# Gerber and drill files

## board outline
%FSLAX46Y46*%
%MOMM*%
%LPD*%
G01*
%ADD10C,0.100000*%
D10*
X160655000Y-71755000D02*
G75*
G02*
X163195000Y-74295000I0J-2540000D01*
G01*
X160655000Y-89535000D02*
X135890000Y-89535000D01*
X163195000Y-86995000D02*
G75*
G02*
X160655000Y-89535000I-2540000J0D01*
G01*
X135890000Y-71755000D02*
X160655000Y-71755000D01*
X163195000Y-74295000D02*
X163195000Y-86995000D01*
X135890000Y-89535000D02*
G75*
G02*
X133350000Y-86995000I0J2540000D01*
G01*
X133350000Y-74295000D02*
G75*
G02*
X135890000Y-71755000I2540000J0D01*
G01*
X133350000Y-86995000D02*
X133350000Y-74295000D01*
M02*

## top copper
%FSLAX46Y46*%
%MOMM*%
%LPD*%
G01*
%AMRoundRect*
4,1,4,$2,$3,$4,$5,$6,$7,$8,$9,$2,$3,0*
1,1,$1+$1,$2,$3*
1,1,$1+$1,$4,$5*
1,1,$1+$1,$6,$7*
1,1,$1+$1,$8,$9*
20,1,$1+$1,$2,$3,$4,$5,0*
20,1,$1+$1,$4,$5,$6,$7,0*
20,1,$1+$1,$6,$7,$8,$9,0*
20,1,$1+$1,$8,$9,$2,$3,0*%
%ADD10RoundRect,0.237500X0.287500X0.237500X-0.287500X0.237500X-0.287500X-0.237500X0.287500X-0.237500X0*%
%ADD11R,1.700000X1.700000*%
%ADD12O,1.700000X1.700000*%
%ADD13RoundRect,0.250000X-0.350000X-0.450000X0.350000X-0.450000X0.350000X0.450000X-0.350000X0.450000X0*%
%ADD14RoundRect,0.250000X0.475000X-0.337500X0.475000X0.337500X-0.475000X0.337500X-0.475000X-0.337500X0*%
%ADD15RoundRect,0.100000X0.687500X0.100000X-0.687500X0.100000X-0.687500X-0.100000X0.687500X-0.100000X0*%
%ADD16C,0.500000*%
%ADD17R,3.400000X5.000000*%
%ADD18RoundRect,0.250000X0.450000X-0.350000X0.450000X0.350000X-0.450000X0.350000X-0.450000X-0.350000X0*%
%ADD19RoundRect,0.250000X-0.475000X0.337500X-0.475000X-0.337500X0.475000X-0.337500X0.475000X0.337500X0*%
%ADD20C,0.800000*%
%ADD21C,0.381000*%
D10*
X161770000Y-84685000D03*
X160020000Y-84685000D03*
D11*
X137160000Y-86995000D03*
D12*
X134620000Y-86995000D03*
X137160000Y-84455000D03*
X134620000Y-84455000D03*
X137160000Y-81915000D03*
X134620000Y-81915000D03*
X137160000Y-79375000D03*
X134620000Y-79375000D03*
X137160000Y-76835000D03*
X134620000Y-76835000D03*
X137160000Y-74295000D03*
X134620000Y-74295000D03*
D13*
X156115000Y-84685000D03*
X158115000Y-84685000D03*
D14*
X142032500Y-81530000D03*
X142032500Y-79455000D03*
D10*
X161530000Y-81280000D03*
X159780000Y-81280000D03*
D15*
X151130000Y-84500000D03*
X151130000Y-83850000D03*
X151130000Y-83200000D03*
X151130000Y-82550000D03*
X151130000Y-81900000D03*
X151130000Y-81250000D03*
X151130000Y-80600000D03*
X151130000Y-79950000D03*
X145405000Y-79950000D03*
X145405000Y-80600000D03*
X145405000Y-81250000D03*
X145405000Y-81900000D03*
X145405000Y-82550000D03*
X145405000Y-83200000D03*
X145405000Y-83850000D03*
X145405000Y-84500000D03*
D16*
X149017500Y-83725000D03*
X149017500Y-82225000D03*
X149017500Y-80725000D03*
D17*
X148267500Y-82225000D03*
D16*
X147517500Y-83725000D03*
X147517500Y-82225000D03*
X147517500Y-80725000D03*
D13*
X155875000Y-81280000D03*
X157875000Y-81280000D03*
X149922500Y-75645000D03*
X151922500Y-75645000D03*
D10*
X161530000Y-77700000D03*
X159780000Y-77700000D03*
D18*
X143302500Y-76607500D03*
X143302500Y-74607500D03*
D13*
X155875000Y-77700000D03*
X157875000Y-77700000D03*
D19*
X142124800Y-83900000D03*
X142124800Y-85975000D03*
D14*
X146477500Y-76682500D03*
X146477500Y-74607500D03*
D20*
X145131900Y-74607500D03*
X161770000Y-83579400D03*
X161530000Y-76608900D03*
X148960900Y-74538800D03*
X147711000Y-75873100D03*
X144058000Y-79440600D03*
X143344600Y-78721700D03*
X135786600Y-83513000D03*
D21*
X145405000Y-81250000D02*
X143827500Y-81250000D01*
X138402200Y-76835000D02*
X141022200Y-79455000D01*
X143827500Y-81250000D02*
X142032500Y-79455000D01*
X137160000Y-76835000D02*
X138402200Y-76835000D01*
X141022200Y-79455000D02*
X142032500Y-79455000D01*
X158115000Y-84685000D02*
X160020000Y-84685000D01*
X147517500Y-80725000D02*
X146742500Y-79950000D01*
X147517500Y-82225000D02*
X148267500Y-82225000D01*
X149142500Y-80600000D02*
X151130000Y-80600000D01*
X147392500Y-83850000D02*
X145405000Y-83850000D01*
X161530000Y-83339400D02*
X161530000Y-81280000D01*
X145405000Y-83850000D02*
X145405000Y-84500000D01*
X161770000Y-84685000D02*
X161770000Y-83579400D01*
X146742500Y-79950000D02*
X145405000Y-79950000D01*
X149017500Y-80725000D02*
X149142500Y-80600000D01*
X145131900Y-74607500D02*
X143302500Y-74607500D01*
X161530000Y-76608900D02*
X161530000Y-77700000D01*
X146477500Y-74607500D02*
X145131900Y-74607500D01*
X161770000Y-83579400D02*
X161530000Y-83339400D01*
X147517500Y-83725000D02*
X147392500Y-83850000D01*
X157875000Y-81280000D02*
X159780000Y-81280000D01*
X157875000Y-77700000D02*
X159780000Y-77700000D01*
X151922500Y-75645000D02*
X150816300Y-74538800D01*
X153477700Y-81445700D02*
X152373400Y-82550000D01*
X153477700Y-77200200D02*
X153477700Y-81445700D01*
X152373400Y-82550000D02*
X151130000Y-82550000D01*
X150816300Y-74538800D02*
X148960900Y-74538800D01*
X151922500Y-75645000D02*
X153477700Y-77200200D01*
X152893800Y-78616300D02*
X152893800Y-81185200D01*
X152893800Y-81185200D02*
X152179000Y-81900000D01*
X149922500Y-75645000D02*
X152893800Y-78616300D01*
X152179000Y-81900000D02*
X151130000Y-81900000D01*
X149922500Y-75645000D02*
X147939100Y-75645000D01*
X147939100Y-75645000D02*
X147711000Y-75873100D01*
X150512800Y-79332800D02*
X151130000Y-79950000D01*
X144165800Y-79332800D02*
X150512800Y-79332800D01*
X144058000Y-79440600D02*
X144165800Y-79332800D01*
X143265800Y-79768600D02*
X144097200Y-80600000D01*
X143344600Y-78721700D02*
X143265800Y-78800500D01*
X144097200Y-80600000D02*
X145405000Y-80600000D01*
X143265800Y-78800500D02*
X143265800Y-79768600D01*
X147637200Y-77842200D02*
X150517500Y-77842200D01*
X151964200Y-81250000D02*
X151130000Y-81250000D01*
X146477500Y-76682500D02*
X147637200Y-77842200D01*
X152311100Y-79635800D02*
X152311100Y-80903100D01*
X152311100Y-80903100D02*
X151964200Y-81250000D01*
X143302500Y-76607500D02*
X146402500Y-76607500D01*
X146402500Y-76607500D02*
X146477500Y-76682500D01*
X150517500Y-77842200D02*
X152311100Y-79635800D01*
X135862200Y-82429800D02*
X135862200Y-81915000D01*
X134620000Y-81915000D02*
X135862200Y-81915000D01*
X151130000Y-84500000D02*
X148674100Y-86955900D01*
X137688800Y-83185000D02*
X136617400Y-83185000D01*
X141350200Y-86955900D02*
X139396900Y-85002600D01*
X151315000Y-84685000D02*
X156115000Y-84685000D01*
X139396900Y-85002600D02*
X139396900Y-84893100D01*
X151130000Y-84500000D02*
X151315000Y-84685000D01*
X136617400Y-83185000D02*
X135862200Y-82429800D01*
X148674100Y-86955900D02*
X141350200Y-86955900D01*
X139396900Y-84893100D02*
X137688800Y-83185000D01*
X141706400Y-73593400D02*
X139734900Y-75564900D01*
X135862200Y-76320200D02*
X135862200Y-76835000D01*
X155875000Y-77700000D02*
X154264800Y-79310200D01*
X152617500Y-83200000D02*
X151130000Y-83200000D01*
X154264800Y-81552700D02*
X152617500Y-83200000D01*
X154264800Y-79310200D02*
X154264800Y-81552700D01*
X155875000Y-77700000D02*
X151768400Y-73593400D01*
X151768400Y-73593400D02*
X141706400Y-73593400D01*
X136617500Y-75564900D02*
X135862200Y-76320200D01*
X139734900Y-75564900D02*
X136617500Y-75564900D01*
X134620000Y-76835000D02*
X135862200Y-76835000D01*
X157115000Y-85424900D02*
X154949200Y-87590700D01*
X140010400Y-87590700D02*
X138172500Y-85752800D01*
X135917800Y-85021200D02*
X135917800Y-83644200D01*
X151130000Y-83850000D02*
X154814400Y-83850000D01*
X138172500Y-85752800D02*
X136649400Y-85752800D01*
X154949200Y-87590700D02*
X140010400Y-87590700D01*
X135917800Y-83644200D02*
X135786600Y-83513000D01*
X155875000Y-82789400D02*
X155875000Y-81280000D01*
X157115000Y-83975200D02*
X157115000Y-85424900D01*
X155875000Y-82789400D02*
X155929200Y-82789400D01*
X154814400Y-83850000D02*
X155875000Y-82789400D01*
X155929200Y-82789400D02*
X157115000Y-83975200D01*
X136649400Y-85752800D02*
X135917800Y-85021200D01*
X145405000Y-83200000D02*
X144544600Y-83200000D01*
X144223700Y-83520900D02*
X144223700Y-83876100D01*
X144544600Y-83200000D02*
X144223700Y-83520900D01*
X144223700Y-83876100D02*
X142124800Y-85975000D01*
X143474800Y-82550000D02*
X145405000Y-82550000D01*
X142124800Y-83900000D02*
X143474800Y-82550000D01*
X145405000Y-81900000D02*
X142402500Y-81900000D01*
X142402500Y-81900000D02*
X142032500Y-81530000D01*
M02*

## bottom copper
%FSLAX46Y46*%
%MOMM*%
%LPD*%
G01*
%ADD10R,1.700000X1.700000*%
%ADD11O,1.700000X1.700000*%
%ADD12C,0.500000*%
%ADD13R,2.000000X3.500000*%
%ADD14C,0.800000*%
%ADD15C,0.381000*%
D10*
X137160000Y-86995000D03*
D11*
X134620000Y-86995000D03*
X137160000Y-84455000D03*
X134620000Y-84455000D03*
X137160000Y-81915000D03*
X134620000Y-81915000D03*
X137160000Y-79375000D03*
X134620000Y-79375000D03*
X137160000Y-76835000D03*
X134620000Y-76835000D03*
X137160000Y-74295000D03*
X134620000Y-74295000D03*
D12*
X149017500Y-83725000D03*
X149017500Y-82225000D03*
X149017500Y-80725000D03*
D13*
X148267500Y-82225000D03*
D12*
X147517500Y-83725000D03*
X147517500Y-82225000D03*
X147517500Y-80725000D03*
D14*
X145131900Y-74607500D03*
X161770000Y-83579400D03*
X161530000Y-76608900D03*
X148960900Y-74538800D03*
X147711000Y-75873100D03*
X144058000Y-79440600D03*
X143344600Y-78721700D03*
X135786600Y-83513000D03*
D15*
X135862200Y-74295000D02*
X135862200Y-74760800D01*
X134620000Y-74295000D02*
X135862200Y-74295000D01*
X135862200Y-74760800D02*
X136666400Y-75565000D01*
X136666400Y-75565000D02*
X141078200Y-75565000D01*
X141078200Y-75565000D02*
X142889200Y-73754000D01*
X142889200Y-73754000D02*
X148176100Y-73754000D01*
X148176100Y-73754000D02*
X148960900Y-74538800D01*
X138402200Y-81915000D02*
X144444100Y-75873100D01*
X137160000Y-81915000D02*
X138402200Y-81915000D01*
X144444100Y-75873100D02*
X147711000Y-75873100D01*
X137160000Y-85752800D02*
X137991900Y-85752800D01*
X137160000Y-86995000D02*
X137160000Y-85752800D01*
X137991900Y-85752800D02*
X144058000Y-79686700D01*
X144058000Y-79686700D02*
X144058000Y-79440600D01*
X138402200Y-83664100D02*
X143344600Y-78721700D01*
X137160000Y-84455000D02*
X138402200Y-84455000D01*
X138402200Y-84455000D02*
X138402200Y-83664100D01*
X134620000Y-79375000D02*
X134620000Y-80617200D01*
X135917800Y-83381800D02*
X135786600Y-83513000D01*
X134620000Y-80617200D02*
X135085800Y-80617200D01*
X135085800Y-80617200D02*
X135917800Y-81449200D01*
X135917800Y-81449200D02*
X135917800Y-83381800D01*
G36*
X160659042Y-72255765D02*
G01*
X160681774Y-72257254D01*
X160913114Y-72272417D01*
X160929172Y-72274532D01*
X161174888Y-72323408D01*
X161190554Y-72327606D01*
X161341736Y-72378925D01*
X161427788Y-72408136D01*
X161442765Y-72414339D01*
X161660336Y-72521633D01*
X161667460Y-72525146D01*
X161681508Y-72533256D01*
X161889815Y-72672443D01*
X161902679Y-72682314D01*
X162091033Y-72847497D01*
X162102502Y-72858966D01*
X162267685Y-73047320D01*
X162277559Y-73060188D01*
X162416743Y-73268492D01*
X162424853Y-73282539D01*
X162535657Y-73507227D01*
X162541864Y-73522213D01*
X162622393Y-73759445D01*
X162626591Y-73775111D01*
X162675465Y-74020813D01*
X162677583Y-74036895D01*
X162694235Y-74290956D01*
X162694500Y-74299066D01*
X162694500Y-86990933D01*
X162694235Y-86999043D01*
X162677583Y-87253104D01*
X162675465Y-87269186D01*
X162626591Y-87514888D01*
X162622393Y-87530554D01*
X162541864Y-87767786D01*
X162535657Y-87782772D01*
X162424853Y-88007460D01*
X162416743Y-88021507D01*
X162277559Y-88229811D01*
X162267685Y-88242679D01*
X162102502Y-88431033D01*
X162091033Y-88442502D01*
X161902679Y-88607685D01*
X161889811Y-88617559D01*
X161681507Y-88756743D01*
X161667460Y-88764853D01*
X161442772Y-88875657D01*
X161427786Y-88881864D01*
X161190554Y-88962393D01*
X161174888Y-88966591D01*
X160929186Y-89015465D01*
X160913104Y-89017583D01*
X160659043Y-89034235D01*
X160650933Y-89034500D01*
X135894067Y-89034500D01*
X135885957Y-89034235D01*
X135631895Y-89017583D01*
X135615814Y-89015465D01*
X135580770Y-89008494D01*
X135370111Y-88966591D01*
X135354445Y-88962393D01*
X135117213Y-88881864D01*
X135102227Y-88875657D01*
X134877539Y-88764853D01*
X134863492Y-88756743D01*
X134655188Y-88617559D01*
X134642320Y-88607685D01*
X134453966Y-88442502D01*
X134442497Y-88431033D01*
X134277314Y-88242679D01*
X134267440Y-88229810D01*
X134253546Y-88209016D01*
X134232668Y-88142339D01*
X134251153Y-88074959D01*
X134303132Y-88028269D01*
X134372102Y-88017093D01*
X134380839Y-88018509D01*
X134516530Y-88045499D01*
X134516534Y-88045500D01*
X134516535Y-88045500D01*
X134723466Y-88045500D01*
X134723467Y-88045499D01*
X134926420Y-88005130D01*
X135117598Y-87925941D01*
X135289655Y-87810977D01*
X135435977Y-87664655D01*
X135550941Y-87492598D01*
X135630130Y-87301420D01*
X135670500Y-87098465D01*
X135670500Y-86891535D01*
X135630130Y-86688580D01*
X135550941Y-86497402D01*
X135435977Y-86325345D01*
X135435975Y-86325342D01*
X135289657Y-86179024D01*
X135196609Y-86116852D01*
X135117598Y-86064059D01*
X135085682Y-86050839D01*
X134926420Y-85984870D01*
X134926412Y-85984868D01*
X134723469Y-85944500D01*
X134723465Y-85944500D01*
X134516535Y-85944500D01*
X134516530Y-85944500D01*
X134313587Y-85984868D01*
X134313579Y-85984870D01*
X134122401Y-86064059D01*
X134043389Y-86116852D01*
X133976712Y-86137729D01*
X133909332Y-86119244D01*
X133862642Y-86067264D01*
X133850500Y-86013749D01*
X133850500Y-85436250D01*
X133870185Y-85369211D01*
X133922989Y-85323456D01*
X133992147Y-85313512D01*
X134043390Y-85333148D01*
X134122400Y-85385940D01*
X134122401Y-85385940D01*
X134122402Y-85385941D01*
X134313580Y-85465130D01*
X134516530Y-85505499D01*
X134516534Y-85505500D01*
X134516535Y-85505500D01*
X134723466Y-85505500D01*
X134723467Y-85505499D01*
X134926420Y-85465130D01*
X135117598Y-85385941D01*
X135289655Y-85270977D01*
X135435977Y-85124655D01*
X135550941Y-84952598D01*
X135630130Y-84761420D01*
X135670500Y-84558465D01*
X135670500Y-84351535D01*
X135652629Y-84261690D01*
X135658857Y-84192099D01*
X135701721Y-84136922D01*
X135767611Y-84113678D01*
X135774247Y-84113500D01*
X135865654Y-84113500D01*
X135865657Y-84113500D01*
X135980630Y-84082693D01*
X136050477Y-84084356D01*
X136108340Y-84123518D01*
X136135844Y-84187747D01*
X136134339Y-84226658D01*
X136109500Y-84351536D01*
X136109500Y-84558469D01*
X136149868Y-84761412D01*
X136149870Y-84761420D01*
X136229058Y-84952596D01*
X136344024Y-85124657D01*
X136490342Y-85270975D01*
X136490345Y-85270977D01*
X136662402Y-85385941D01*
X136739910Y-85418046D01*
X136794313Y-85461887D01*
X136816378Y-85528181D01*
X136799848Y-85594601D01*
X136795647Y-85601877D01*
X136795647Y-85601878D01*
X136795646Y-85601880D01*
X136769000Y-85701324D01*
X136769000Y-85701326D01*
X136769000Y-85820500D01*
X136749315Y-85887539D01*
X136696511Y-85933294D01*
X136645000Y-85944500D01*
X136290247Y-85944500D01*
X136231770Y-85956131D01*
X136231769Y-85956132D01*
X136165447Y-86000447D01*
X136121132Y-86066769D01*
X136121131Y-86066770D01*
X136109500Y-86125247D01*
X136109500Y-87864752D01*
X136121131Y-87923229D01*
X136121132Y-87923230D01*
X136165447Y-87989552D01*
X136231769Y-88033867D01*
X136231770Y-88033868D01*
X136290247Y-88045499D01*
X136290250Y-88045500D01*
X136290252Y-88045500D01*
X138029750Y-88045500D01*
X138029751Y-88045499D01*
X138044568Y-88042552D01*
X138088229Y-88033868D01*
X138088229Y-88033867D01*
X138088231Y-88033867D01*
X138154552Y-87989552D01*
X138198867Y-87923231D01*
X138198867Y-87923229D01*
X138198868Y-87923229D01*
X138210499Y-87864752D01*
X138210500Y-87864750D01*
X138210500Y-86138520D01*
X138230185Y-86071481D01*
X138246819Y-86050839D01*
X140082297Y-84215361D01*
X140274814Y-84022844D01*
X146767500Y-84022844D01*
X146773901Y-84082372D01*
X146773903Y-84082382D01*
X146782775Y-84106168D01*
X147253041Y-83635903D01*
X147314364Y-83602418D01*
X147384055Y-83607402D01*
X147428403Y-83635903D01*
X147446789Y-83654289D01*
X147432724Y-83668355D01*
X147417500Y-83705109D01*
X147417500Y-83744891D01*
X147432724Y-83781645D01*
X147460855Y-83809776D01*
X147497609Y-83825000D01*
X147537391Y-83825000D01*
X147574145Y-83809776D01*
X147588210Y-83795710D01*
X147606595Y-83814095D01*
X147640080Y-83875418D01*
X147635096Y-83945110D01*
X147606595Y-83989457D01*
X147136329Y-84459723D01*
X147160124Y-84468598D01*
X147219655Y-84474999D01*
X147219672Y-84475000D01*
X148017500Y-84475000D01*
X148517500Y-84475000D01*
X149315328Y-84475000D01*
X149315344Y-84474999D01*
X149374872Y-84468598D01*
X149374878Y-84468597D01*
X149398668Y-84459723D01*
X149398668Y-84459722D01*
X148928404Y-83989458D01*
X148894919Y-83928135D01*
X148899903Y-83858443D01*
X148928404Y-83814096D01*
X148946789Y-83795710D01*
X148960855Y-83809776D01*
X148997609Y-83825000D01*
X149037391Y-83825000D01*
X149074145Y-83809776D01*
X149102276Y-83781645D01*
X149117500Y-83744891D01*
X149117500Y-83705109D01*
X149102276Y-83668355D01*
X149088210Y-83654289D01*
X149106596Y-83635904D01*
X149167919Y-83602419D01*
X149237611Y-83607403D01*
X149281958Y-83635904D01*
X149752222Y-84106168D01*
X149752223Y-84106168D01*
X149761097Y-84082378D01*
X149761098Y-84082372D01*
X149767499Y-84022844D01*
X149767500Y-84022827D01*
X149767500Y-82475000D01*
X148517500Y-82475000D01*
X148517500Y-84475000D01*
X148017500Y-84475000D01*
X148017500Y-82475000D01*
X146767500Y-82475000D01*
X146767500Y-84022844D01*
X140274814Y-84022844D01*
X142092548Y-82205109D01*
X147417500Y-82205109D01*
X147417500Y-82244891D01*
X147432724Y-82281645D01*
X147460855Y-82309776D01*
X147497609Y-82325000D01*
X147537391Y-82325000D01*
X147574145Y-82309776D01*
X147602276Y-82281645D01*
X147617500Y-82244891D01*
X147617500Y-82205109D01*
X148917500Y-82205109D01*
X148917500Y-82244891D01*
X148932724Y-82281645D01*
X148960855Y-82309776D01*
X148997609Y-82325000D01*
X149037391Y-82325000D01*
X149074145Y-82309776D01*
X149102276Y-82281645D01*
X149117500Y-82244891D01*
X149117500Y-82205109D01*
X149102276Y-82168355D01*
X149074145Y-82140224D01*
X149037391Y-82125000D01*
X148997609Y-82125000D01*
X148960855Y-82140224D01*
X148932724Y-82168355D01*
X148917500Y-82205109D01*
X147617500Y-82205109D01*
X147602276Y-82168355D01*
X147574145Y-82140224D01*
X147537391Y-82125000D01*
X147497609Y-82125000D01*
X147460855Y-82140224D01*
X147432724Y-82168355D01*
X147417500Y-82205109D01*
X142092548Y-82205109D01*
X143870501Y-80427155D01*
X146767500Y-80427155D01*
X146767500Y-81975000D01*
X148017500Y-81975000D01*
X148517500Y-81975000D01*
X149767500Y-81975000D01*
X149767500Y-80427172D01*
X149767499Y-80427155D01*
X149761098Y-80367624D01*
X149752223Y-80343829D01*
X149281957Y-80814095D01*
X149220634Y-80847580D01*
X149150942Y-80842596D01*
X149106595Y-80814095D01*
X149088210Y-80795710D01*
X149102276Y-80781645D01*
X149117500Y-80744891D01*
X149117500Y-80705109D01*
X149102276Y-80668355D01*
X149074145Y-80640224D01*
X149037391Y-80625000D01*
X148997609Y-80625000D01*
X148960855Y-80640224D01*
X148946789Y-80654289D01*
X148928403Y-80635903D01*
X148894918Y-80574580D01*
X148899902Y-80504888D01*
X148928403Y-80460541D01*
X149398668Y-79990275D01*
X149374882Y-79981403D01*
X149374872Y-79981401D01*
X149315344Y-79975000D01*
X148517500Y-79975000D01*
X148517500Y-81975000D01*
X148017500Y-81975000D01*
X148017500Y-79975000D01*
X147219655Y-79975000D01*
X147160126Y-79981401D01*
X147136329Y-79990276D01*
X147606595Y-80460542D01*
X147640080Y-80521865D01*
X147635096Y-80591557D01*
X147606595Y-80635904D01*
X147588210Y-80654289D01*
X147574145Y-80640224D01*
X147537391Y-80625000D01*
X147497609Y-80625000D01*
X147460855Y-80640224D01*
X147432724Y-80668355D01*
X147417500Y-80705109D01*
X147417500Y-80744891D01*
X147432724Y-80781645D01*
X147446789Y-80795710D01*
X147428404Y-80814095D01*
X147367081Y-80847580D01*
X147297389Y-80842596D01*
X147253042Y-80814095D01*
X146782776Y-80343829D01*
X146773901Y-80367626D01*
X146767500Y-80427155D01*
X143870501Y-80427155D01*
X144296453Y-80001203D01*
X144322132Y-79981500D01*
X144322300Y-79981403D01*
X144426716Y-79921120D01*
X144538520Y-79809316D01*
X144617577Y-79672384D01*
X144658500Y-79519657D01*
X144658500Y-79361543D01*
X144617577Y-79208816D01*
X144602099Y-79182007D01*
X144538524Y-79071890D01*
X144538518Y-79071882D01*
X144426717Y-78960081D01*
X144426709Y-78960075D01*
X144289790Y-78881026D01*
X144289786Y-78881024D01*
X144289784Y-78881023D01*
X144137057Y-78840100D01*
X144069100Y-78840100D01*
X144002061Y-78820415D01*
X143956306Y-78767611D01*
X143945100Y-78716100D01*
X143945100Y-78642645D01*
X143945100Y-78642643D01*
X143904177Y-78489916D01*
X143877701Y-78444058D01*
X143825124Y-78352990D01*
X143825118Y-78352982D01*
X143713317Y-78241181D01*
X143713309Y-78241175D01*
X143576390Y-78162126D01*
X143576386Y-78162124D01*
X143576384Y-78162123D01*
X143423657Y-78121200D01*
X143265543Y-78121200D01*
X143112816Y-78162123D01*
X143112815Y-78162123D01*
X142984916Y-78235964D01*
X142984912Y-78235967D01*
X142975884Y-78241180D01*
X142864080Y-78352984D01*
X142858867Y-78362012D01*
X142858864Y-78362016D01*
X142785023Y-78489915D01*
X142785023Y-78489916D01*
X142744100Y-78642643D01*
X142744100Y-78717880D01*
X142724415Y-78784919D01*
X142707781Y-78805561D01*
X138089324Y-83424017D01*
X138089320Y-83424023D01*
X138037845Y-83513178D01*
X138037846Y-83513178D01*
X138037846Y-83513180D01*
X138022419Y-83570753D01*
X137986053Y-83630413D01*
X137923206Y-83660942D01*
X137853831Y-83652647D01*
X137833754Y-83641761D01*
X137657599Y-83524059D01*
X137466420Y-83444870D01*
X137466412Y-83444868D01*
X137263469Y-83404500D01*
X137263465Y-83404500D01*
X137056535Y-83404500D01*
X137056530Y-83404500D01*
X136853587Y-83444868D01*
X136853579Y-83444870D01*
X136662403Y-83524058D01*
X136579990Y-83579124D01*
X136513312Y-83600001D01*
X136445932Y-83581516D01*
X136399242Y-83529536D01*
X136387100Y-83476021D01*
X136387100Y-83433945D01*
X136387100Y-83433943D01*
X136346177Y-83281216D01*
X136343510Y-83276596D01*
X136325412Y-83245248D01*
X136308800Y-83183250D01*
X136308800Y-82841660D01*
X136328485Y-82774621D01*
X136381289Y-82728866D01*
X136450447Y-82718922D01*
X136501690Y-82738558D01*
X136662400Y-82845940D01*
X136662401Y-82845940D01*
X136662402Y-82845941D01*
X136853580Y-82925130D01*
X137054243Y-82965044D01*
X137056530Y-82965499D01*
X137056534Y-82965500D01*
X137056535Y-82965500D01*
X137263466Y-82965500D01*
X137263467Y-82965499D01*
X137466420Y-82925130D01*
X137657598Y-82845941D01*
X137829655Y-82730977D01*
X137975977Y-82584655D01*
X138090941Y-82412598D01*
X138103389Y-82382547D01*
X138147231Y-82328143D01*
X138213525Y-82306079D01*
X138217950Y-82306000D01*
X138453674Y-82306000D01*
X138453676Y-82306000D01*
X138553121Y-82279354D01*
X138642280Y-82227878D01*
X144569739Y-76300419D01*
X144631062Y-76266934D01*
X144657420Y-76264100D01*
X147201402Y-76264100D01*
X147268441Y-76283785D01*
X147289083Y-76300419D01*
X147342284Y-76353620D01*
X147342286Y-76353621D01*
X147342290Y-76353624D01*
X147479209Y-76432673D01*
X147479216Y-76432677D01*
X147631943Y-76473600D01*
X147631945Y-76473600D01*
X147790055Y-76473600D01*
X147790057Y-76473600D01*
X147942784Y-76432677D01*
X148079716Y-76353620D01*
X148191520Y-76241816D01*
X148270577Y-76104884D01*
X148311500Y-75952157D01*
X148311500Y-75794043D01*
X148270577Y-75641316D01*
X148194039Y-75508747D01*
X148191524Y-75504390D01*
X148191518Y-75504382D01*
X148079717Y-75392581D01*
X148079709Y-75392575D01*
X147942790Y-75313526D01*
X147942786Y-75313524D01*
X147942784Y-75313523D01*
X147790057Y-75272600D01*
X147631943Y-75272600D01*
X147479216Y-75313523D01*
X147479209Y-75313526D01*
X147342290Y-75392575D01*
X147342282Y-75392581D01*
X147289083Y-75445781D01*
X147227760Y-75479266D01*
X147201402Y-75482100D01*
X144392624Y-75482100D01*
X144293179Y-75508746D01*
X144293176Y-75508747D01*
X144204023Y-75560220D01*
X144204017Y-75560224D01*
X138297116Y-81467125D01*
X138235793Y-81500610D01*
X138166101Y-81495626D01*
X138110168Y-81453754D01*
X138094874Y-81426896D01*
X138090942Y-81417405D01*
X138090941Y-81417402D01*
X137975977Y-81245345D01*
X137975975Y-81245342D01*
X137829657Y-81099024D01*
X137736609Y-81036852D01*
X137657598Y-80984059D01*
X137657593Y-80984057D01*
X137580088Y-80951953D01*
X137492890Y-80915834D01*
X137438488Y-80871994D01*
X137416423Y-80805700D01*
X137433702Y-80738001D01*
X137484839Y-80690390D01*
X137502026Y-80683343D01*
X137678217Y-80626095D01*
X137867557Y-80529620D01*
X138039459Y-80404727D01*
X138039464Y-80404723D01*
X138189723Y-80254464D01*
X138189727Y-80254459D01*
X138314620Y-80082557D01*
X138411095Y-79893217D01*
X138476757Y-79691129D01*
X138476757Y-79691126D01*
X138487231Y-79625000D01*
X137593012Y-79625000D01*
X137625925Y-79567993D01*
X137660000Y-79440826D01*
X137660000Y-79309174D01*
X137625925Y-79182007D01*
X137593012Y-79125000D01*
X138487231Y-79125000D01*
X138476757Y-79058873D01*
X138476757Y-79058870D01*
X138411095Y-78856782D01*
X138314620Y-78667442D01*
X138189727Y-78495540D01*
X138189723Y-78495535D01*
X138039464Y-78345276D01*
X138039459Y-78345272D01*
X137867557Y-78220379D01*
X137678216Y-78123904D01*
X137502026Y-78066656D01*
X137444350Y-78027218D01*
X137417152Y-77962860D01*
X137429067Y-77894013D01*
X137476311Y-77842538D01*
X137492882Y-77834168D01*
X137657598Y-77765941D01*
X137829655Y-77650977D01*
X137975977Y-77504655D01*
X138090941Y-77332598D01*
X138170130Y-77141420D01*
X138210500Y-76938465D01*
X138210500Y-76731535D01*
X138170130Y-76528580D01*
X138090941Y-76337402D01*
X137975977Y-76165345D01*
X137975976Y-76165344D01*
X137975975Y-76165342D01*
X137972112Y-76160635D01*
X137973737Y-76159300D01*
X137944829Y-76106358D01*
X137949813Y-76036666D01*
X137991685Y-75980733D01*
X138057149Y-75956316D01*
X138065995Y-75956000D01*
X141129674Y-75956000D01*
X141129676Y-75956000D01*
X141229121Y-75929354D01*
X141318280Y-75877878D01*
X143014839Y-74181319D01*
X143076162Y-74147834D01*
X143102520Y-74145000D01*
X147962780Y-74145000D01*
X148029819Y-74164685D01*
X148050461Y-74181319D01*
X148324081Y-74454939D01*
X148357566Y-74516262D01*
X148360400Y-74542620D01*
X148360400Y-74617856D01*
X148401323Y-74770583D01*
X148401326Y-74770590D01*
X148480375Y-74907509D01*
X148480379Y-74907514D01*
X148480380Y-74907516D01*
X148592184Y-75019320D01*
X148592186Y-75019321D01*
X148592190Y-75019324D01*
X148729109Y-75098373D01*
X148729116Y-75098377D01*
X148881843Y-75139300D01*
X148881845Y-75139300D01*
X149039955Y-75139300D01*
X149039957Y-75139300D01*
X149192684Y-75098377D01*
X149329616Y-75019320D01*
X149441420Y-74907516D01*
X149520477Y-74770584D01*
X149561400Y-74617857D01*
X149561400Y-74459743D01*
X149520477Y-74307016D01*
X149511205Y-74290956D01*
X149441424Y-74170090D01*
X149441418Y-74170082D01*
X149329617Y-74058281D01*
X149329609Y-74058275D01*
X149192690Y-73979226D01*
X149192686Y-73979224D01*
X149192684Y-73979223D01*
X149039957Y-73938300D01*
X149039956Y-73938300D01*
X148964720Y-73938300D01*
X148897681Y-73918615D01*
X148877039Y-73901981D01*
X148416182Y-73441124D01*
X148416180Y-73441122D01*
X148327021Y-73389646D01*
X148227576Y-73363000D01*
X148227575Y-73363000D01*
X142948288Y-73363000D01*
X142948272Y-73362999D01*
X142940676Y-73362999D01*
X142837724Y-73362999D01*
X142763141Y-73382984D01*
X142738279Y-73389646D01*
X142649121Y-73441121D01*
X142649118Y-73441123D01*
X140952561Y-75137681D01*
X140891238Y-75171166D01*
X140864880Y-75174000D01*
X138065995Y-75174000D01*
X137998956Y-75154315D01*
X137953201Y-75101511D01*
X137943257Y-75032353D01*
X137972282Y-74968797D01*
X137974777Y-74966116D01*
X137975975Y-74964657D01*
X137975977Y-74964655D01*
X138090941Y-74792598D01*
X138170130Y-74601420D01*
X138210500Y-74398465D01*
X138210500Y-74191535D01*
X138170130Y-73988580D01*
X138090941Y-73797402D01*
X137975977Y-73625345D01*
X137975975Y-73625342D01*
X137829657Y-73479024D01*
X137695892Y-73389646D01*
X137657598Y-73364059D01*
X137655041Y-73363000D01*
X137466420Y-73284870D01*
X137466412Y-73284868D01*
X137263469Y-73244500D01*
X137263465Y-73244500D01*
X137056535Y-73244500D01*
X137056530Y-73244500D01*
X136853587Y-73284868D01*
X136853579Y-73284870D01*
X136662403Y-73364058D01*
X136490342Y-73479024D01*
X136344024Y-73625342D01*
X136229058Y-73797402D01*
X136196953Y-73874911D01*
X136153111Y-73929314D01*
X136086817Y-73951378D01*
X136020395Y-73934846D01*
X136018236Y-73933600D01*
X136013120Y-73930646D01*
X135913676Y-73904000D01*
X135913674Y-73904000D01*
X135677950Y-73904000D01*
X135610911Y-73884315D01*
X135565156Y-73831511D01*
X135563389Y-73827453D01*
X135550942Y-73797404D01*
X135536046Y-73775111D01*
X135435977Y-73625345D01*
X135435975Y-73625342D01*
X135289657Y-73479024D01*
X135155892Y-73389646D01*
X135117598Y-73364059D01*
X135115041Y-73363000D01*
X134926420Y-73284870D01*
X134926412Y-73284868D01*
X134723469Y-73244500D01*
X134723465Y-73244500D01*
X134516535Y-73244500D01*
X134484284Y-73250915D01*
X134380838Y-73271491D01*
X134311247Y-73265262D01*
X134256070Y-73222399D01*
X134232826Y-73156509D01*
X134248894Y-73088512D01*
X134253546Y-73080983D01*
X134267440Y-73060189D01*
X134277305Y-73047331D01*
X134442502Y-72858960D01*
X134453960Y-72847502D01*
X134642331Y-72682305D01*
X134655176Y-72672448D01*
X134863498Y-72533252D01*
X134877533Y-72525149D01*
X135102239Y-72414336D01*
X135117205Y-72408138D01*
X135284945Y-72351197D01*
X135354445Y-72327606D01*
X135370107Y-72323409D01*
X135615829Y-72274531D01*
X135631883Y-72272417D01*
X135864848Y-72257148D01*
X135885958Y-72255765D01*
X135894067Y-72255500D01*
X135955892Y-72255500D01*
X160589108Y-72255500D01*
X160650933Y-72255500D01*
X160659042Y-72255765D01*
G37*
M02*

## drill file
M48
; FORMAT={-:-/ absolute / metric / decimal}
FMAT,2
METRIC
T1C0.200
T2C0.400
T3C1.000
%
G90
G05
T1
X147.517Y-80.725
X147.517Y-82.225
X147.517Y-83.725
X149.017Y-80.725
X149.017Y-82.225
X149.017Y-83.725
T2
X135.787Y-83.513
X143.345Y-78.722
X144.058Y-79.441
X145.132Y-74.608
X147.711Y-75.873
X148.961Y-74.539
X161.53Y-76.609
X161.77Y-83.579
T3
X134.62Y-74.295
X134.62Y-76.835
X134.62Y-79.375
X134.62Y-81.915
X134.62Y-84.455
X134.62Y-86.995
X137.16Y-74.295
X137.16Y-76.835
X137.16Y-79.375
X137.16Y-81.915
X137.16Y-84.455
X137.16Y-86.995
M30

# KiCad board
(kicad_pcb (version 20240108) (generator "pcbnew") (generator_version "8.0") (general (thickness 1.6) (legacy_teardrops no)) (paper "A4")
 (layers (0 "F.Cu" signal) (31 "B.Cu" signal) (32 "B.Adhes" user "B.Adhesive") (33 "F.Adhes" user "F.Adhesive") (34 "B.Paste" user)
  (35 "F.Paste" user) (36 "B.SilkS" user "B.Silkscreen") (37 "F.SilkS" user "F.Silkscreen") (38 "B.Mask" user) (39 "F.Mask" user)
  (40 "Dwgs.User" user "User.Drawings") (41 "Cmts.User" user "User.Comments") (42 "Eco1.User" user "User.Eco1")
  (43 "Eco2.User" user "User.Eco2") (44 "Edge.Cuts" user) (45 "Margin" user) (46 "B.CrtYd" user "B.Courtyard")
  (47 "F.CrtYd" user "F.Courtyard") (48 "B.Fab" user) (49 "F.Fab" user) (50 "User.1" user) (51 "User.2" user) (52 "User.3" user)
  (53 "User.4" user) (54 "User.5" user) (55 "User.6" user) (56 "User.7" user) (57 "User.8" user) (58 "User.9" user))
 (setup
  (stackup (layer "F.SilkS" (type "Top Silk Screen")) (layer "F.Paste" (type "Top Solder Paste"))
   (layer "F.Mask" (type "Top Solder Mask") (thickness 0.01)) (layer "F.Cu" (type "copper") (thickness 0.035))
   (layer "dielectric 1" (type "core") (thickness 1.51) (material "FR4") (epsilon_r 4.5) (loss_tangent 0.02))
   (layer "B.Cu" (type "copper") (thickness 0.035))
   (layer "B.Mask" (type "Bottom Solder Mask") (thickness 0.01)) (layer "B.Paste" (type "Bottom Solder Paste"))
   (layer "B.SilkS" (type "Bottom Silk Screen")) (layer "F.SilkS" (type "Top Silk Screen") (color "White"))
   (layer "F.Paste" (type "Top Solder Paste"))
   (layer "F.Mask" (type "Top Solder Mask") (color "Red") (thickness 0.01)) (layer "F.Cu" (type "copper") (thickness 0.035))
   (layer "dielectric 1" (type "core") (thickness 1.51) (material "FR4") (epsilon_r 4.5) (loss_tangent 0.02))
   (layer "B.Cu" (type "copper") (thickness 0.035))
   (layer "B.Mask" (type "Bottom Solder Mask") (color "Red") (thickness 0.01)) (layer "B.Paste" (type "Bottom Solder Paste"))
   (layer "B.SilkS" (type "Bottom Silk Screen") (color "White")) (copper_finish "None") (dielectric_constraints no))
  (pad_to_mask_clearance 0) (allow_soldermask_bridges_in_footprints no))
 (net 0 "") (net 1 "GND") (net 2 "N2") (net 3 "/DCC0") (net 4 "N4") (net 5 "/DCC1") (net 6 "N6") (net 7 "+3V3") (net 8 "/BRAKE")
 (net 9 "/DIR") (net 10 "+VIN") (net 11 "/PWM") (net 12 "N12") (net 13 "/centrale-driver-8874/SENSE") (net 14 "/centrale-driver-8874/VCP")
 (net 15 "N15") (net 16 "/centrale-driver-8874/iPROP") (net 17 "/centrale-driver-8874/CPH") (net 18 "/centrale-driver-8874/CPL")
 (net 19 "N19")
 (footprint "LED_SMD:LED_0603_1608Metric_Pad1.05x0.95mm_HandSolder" (layer "F.Cu") (at 160.895 84.685 180)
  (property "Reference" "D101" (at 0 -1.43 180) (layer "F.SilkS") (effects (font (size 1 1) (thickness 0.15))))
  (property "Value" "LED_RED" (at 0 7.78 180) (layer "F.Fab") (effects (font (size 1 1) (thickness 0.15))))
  (pad "1" smd roundrect (at -0.875 0 180) (size 1.05 0.95) (layers "F.Cu" "F.Paste" "F.Mask") (roundrect_rratio 0.25) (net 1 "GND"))
  (pad "2" smd roundrect (at 0.875 0 180) (size 1.05 0.95) (layers "F.Cu" "F.Paste" "F.Mask") (roundrect_rratio 0.25) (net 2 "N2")))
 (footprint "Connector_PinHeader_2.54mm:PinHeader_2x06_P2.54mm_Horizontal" (layer "F.Cu") (at 137.16 86.995 180)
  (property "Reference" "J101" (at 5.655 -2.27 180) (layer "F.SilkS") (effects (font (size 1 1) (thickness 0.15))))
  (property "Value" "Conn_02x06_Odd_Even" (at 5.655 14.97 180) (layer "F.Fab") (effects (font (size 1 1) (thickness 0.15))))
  (pad "1" thru_hole rect (at 0 0 180) (size 1.7 1.7) (drill 1) (layers "*.Cu" "*.Mask") (remove_unused_layers no) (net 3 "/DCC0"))
  (pad "2" thru_hole oval (at 2.54 0 180) (size 1.7 1.7) (drill 1) (layers "*.Cu" "*.Mask") (remove_unused_layers no) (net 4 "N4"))
  (pad "3" thru_hole oval (at 0 2.54 180) (size 1.7 1.7) (drill 1) (layers "*.Cu" "*.Mask") (remove_unused_layers no) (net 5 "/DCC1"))
  (pad "4" thru_hole oval (at 2.54 2.54 180) (size 1.7 1.7) (drill 1) (layers "*.Cu" "*.Mask") (remove_unused_layers no) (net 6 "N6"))
  (pad "5" thru_hole oval (at 0 5.08 180) (size 1.7 1.7) (drill 1) (layers "*.Cu" "*.Mask") (remove_unused_layers no) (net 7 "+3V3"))
  (pad "6" thru_hole oval (at 2.54 5.08 180) (size 1.7 1.7) (drill 1) (layers "*.Cu" "*.Mask") (remove_unused_layers no) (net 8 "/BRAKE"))
  (pad "7" thru_hole oval (at 0 7.62 180) (size 1.7 1.7) (drill 1) (layers "*.Cu" "*.Mask") (remove_unused_layers no) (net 1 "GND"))
  (pad "8" thru_hole oval (at 2.54 7.62 180) (size 1.7 1.7) (drill 1) (layers "*.Cu" "*.Mask") (remove_unused_layers no) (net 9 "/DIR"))
  (pad "9" thru_hole oval (at 0 10.16 180) (size 1.7 1.7) (drill 1) (layers "*.Cu" "*.Mask") (remove_unused_layers no) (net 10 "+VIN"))
  (pad "10" thru_hole oval (at 2.54 10.16 180) (size 1.7 1.7) (drill 1) (layers "*.Cu" "*.Mask") (remove_unused_layers no) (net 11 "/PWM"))
  (pad "11" thru_hole oval (at 0 12.7 180) (size 1.7 1.7) (drill 1) (layers "*.Cu" "*.Mask") (remove_unused_layers no) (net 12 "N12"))
  (pad "12" thru_hole oval (at 2.54 12.7 180) (size 1.7 1.7) (drill 1) (layers "*.Cu" "*.Mask") (remove_unused_layers no)
   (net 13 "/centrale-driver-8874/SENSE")))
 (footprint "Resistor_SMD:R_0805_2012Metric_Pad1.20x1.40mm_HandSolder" (layer "F.Cu") (at 157.115 84.685)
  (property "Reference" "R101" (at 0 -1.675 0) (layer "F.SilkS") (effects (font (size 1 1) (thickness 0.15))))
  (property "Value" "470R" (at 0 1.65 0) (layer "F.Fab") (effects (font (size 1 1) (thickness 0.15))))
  (pad "1" smd roundrect (at -1 0) (size 1.2 1.4) (layers "F.Cu" "F.Paste" "F.Mask") (roundrect_rratio 0.208333) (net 8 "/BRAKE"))
  (pad "2" smd roundrect (at 1 0) (size 1.2 1.4) (layers "F.Cu" "F.Paste" "F.Mask") (roundrect_rratio 0.208333) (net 2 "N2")))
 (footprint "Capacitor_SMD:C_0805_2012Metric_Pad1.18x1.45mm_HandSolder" (layer "F.Cu") (at 142.0325 80.4925 90)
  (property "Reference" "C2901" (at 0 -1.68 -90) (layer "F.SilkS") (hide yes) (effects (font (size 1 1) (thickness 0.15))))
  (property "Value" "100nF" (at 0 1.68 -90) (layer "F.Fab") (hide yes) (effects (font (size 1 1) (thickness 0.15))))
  (pad "1" smd roundrect (at -1.0375 0 90) (size 1.175 1.45) (layers "F.Cu" "F.Paste" "F.Mask") (roundrect_rratio 0.212766)
   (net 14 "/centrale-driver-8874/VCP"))
  (pad "2" smd roundrect (at 1.0375 0 90) (size 1.175 1.45) (layers "F.Cu" "F.Paste" "F.Mask") (roundrect_rratio 0.212766) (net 10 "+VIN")))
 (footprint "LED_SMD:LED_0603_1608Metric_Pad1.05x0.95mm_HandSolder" (layer "F.Cu") (at 160.655 81.28 180)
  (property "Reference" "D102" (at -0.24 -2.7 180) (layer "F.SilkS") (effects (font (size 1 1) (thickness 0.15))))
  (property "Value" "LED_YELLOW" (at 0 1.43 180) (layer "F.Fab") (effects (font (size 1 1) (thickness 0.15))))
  (pad "1" smd roundrect (at -0.875 0 180) (size 1.05 0.95) (layers "F.Cu" "F.Paste" "F.Mask") (roundrect_rratio 0.25) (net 1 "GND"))
  (pad "2" smd roundrect (at 0.875 0 180) (size 1.05 0.95) (layers "F.Cu" "F.Paste" "F.Mask") (roundrect_rratio 0.25) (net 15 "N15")))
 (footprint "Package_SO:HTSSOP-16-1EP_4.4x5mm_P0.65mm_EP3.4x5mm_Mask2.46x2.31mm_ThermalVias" (layer "F.Cu") (at 148.2675 82.225 180)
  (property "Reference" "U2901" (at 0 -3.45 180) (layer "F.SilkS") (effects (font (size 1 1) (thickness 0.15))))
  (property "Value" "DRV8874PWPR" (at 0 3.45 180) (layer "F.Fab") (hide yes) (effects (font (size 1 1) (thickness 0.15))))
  (pad "" smd roundrect (at 0 -0.58 180) (size 1.98 0.93) (layers "F.Paste") (roundrect_rratio 0.25))
  (pad "" smd rect (at 0 0 180) (size 2.46 2.31) (layers "F.Mask"))
  (pad "" smd roundrect (at 0 0.58 180) (size 1.98 0.93) (layers "F.Paste") (roundrect_rratio 0.25))
  (pad "1" smd roundrect (at -2.8625 -2.275 180) (size 1.575 0.4) (layers "F.Cu" "F.Paste" "F.Mask") (roundrect_rratio 0.25)
   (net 8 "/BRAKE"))
  (pad "2" smd roundrect (at -2.8625 -1.625 180) (size 1.575 0.4) (layers "F.Cu" "F.Paste" "F.Mask") (roundrect_rratio 0.25) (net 9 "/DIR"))
  (pad "3" smd roundrect (at -2.8625 -0.975 180) (size 1.575 0.4) (layers "F.Cu" "F.Paste" "F.Mask") (roundrect_rratio 0.25) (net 11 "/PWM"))
  (pad "4" smd roundrect (at -2.8625 -0.325 180) (size 1.575 0.4) (layers "F.Cu" "F.Paste" "F.Mask") (roundrect_rratio 0.25)
   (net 13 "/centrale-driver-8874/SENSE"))
  (pad "5" smd roundrect (at -2.8625 0.325 180) (size 1.575 0.4) (layers "F.Cu" "F.Paste" "F.Mask") (roundrect_rratio 0.25) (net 7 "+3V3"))
  (pad "6" smd roundrect (at -2.8625 0.975 180) (size 1.575 0.4) (layers "F.Cu" "F.Paste" "F.Mask") (roundrect_rratio 0.25)
   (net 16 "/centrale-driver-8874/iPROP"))
  (pad "7" smd roundrect (at -2.8625 1.625 180) (size 1.575 0.4) (layers "F.Cu" "F.Paste" "F.Mask") (roundrect_rratio 0.25) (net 1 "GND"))
  (pad "8" smd roundrect (at -2.8625 2.275 180) (size 1.575 0.4) (layers "F.Cu" "F.Paste" "F.Mask") (roundrect_rratio 0.25) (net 3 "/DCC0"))
  (pad "9" smd roundrect (at 2.8625 2.275 180) (size 1.575 0.4) (layers "F.Cu" "F.Paste" "F.Mask") (roundrect_rratio 0.25) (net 1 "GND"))
  (pad "10" smd roundrect (at 2.8625 1.625 180) (size 1.575 0.4) (layers "F.Cu" "F.Paste" "F.Mask") (roundrect_rratio 0.25) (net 5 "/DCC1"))
  (pad "11" smd roundrect (at 2.8625 0.975 180) (size 1.575 0.4) (layers "F.Cu" "F.Paste" "F.Mask") (roundrect_rratio 0.25) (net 10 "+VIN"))
  (pad "12" smd roundrect (at 2.8625 0.325 180) (size 1.575 0.4) (layers "F.Cu" "F.Paste" "F.Mask") (roundrect_rratio 0.25)
   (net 14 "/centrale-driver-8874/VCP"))
  (pad "13" smd roundrect (at 2.8625 -0.325 180) (size 1.575 0.4) (layers "F.Cu" "F.Paste" "F.Mask") (roundrect_rratio 0.25)
   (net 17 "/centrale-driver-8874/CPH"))
  (pad "14" smd roundrect (at 2.8625 -0.975 180) (size 1.575 0.4) (layers "F.Cu" "F.Paste" "F.Mask") (roundrect_rratio 0.25)
   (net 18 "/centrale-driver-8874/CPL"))
  (pad "15" smd roundrect (at 2.8625 -1.625 180) (size 1.575 0.4) (layers "F.Cu" "F.Paste" "F.Mask") (roundrect_rratio 0.25) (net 1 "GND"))
  (pad "16" smd roundrect (at 2.8625 -2.275 180) (size 1.575 0.4) (layers "F.Cu" "F.Paste" "F.Mask") (roundrect_rratio 0.25) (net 1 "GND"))
  (pad "17" thru_hole circle (at -0.75 -1.5 180) (size 0.5 0.5) (drill 0.2) (layers "*.Cu") (remove_unused_layers no) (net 1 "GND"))
  (pad "17" thru_hole circle (at -0.75 0 180) (size 0.5 0.5) (drill 0.2) (layers "*.Cu") (remove_unused_layers no) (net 1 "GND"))
  (pad "17" thru_hole circle (at -0.75 1.5 180) (size 0.5 0.5) (drill 0.2) (layers "*.Cu") (remove_unused_layers no) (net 1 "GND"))
  (pad "17" smd rect (at 0 0 180) (size 2 3.5) (layers "B.Cu") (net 1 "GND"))
  (pad "17" smd rect (at 0 0 180) (size 3.4 5) (layers "F.Cu") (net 1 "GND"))
  (pad "17" thru_hole circle (at 0.75 -1.5 180) (size 0.5 0.5) (drill 0.2) (layers "*.Cu") (remove_unused_layers no) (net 1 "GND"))
  (pad "17" thru_hole circle (at 0.75 0 180) (size 0.5 0.5) (drill 0.2) (layers "*.Cu") (remove_unused_layers no) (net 1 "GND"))
  (pad "17" thru_hole circle (at 0.75 1.5 180) (size 0.5 0.5) (drill 0.2) (layers "*.Cu") (remove_unused_layers no) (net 1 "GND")))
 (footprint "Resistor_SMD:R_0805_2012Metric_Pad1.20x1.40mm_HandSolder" (layer "F.Cu") (at 156.875 81.28)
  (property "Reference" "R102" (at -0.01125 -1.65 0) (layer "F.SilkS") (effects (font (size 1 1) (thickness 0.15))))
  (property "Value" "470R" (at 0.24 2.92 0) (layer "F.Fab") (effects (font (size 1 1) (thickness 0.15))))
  (pad "1" smd roundrect (at -1 0) (size 1.2 1.4) (layers "F.Cu" "F.Paste" "F.Mask") (roundrect_rratio 0.208333) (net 9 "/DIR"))
  (pad "2" smd roundrect (at 1 0) (size 1.2 1.4) (layers "F.Cu" "F.Paste" "F.Mask") (roundrect_rratio 0.208333) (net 15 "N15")))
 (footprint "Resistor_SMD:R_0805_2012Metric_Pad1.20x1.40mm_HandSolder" (layer "F.Cu") (at 150.9225 75.645)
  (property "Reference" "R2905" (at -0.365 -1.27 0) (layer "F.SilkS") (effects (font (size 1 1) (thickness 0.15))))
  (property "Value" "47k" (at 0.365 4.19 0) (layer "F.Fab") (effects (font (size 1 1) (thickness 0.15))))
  (pad "1" smd roundrect (at -1 0) (size 1.2 1.4) (layers "F.Cu" "F.Paste" "F.Mask") (roundrect_rratio 0.208333) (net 7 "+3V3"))
  (pad "2" smd roundrect (at 1 0) (size 1.2 1.4) (layers "F.Cu" "F.Paste" "F.Mask") (roundrect_rratio 0.208333)
   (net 13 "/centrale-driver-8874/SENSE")))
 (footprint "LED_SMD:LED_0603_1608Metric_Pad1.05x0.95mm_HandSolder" (layer "F.Cu") (at 160.655 77.7 180)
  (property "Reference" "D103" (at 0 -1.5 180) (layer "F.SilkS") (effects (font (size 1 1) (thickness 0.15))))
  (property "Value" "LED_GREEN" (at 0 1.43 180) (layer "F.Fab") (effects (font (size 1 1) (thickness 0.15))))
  (pad "1" smd roundrect (at -0.875 0 180) (size 1.05 0.95) (layers "F.Cu" "F.Paste" "F.Mask") (roundrect_rratio 0.25) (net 1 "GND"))
  (pad "2" smd roundrect (at 0.875 0 180) (size 1.05 0.95) (layers "F.Cu" "F.Paste" "F.Mask") (roundrect_rratio 0.25) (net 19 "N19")))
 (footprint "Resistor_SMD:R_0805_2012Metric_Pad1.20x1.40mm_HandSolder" (layer "F.Cu") (at 143.3025 75.6075 90)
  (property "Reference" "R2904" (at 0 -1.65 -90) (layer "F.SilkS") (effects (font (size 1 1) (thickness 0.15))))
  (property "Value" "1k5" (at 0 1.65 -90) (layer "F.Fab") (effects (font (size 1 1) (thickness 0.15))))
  (pad "1" smd roundrect (at -1 0 90) (size 1.2 1.4) (layers "F.Cu" "F.Paste" "F.Mask") (roundrect_rratio 0.208333)
   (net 16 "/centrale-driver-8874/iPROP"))
  (pad "2" smd roundrect (at 1 0 90) (size 1.2 1.4) (layers "F.Cu" "F.Paste" "F.Mask") (roundrect_rratio 0.208333) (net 1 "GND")))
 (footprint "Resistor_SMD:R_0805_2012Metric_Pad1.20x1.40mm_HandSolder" (layer "F.Cu") (at 156.875 77.7)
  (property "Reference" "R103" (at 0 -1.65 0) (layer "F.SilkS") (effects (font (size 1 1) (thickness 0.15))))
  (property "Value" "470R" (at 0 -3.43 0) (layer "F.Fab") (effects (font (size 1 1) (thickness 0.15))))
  (pad "1" smd roundrect (at -1 0) (size 1.2 1.4) (layers "F.Cu" "F.Paste" "F.Mask") (roundrect_rratio 0.208333) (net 11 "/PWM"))
  (pad "2" smd roundrect (at 1 0) (size 1.2 1.4) (layers "F.Cu" "F.Paste" "F.Mask") (roundrect_rratio 0.208333) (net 19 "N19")))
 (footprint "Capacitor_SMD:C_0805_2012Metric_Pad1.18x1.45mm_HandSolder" (layer "F.Cu") (at 142.1248 84.9375 -90)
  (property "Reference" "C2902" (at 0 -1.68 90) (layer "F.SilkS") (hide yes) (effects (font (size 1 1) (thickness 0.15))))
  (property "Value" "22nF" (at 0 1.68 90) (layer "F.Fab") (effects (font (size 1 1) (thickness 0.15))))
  (pad "1" smd roundrect (at -1.0375 0 270) (size 1.175 1.45) (layers "F.Cu" "F.Paste" "F.Mask") (roundrect_rratio 0.212766)
   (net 17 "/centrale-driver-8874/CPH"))
  (pad "2" smd roundrect (at 1.0375 0 270) (size 1.175 1.45) (layers "F.Cu" "F.Paste" "F.Mask") (roundrect_rratio 0.212766)
   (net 18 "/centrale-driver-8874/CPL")))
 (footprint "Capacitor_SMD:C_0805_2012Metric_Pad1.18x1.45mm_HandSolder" (layer "F.Cu") (at 146.4775 75.645 90)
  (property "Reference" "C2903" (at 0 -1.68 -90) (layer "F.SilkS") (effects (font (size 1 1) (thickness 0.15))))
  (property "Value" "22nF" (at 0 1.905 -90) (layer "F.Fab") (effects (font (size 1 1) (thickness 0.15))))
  (pad "1" smd roundrect (at -1.0375 0 90) (size 1.175 1.45) (layers "F.Cu" "F.Paste" "F.Mask") (roundrect_rratio 0.212766)
   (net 16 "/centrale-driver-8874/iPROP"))
  (pad "2" smd roundrect (at 1.0375 0 90) (size 1.175 1.45) (layers "F.Cu" "F.Paste" "F.Mask") (roundrect_rratio 0.212766) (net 1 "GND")))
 (gr_arc (start 160.655 71.755) (mid 162.451051 72.498949) (end 163.195 74.295) (stroke (width 0.1) (type default)) (layer "Edge.Cuts"))
 (gr_line (start 160.655 89.535) (end 135.89 89.535) (stroke (width 0.1) (type default)) (layer "Edge.Cuts"))
 (gr_arc (start 163.195 86.995) (mid 162.451051 88.791051) (end 160.655 89.535) (stroke (width 0.1) (type default)) (layer "Edge.Cuts"))
 (gr_line (start 135.89 71.755) (end 160.655 71.755) (stroke (width 0.1) (type default)) (layer "Edge.Cuts"))
 (gr_line (start 163.195 74.295) (end 163.195 86.995) (stroke (width 0.1) (type default)) (layer "Edge.Cuts"))
 (gr_arc (start 135.89 89.535) (mid 134.093949 88.791051) (end 133.35 86.995) (stroke (width 0.1) (type default)) (layer "Edge.Cuts"))
 (gr_arc (start 133.35 74.295) (mid 134.093949 72.498949) (end 135.89 71.755) (stroke (width 0.1) (type default)) (layer "Edge.Cuts"))
 (gr_line (start 133.35 86.995) (end 133.35 74.295) (stroke (width 0.1) (type default)) (layer "Edge.Cuts"))
 (segment (start 145.405 81.25) (end 143.8275 81.25) (width 0.381) (layer "F.Cu") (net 10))
 (segment (start 138.4022 76.835) (end 141.0222 79.455) (width 0.381) (layer "F.Cu") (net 10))
 (segment (start 143.8275 81.25) (end 142.0325 79.455) (width 0.381) (layer "F.Cu") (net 10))
 (segment (start 137.16 76.835) (end 138.4022 76.835) (width 0.381) (layer "F.Cu") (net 10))
 (segment (start 141.0222 79.455) (end 142.0325 79.455) (width 0.381) (layer "F.Cu") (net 10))
 (segment (start 158.115 84.685) (end 160.02 84.685) (width 0.381) (layer "F.Cu") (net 2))
 (segment (start 147.5175 80.725) (end 146.7425 79.95) (width 0.381) (layer "F.Cu") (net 1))
 (segment (start 147.5175 82.225) (end 148.2675 82.225) (width 0.381) (layer "F.Cu") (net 1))
 (segment (start 149.1425 80.6) (end 151.13 80.6) (width 0.381) (layer "F.Cu") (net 1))
 (segment (start 147.3925 83.85) (end 145.405 83.85) (width 0.381) (layer "F.Cu") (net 1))
 (segment (start 161.53 83.3394) (end 161.53 81.28) (width 0.381) (layer "F.Cu") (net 1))
 (segment (start 145.405 83.85) (end 145.405 84.5) (width 0.381) (layer "F.Cu") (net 1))
 (segment (start 161.77 84.685) (end 161.77 83.5794) (width 0.381) (layer "F.Cu") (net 1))
 (segment (start 146.7425 79.95) (end 145.405 79.95) (width 0.381) (layer "F.Cu") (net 1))
 (segment (start 149.0175 80.725) (end 149.1425 80.6) (width 0.381) (layer "F.Cu") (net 1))
 (segment (start 145.1319 74.6075) (end 143.3025 74.6075) (width 0.381) (layer "F.Cu") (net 1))
 (segment (start 161.53 76.6089) (end 161.53 77.7) (width 0.381) (layer "F.Cu") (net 1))
 (segment (start 146.4775 74.6075) (end 145.1319 74.6075) (width 0.381) (layer "F.Cu") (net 1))
 (segment (start 161.77 83.5794) (end 161.53 83.3394) (width 0.381) (layer "F.Cu") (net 1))
 (segment (start 147.5175 83.725) (end 147.3925 83.85) (width 0.381) (layer "F.Cu") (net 1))
 (via (at 145.1319 74.6075) (size 0.8) (drill 0.4) (layers "F.Cu" "B.Cu") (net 1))
 (via (at 161.77 83.5794) (size 0.8) (drill 0.4) (layers "F.Cu" "B.Cu") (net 1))
 (via (at 161.53 76.6089) (size 0.8) (drill 0.4) (layers "F.Cu" "B.Cu") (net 1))
 (segment (start 157.875 81.28) (end 159.78 81.28) (width 0.381) (layer "F.Cu") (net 15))
 (segment (start 157.875 77.7) (end 159.78 77.7) (width 0.381) (layer "F.Cu") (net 19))
 (segment (start 151.9225 75.645) (end 150.8163 74.5388) (width 0.381) (layer "F.Cu") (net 13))
 (segment (start 153.4777 81.4457) (end 152.3734 82.55) (width 0.381) (layer "F.Cu") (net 13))
 (segment (start 153.4777 77.2002) (end 153.4777 81.4457) (width 0.381) (layer "F.Cu") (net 13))
 (segment (start 152.3734 82.55) (end 151.13 82.55) (width 0.381) (layer "F.Cu") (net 13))
 (segment (start 150.8163 74.5388) (end 148.9609 74.5388) (width 0.381) (layer "F.Cu") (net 13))
 (segment (start 151.9225 75.645) (end 153.4777 77.2002) (width 0.381) (layer "F.Cu") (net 13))
 (via (at 148.9609 74.5388) (size 0.8) (drill 0.4) (layers "F.Cu" "B.Cu") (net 13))
 (segment (start 135.8622 74.295) (end 135.8622 74.7608) (width 0.381) (layer "B.Cu") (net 13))
 (segment (start 134.62 74.295) (end 135.8622 74.295) (width 0.381) (layer "B.Cu") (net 13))
 (segment (start 135.8622 74.7608) (end 136.6664 75.565) (width 0.381) (layer "B.Cu") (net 13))
 (segment (start 136.6664 75.565) (end 141.0782 75.565) (width 0.381) (layer "B.Cu") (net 13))
 (segment (start 141.0782 75.565) (end 142.8892 73.754) (width 0.381) (layer "B.Cu") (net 13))
 (segment (start 142.8892 73.754) (end 148.1761 73.754) (width 0.381) (layer "B.Cu") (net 13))
 (segment (start 148.1761 73.754) (end 148.9609 74.5388) (width 0.381) (layer "B.Cu") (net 13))
 (segment (start 152.8938 78.6163) (end 152.8938 81.1852) (width 0.381) (layer "F.Cu") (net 7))
 (segment (start 152.8938 81.1852) (end 152.179 81.9) (width 0.381) (layer "F.Cu") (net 7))
 (segment (start 149.9225 75.645) (end 152.8938 78.6163) (width 0.381) (layer "F.Cu") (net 7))
 (segment (start 152.179 81.9) (end 151.13 81.9) (width 0.381) (layer "F.Cu") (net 7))
 (segment (start 149.9225 75.645) (end 147.9391 75.645) (width 0.381) (layer "F.Cu") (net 7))
 (segment (start 147.9391 75.645) (end 147.711 75.8731) (width 0.381) (layer "F.Cu") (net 7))
 (via (at 147.711 75.8731) (size 0.8) (drill 0.4) (layers "F.Cu" "B.Cu") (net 7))
 (segment (start 138.4022 81.915) (end 144.4441 75.8731) (width 0.381) (layer "B.Cu") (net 7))
 (segment (start 137.16 81.915) (end 138.4022 81.915) (width 0.381) (layer "B.Cu") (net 7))
 (segment (start 144.4441 75.8731) (end 147.711 75.8731) (width 0.381) (layer "B.Cu") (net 7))
 (segment (start 150.5128 79.3328) (end 151.13 79.95) (width 0.381) (layer "F.Cu") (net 3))
 (segment (start 144.1658 79.3328) (end 150.5128 79.3328) (width 0.381) (layer "F.Cu") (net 3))
 (segment (start 144.058 79.4406) (end 144.1658 79.3328) (width 0.381) (layer "F.Cu") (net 3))
 (via (at 144.058 79.4406) (size 0.8) (drill 0.4) (layers "F.Cu" "B.Cu") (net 3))
 (segment (start 137.16 85.7528) (end 137.9919 85.7528) (width 0.381) (layer "B.Cu") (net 3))
 (segment (start 137.16 86.995) (end 137.16 85.7528) (width 0.381) (layer "B.Cu") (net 3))
 (segment (start 137.9919 85.7528) (end 144.058 79.6867) (width 0.381) (layer "B.Cu") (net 3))
 (segment (start 144.058 79.6867) (end 144.058 79.4406) (width 0.381) (layer "B.Cu") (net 3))
 (segment (start 143.2658 79.7686) (end 144.0972 80.6) (width 0.381) (layer "F.Cu") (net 5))
 (segment (start 143.3446 78.7217) (end 143.2658 78.8005) (width 0.381) (layer "F.Cu") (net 5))
 (segment (start 144.0972 80.6) (end 145.405 80.6) (width 0.381) (layer "F.Cu") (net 5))
 (segment (start 143.2658 78.8005) (end 143.2658 79.7686) (width 0.381) (layer "F.Cu") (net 5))
 (via (at 143.3446 78.7217) (size 0.8) (drill 0.4) (layers "F.Cu" "B.Cu") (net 5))
 (segment (start 138.4022 83.6641) (end 143.3446 78.7217) (width 0.381) (layer "B.Cu") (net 5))
 (segment (start 137.16 84.455) (end 138.4022 84.455) (width 0.381) (layer "B.Cu") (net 5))
 (segment (start 138.4022 84.455) (end 138.4022 83.6641) (width 0.381) (layer "B.Cu") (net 5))
 (segment (start 147.6372 77.8422) (end 150.5175 77.8422) (width 0.381) (layer "F.Cu") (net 16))
 (segment (start 151.9642 81.25) (end 151.13 81.25) (width 0.381) (layer "F.Cu") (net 16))
 (segment (start 146.4775 76.6825) (end 147.6372 77.8422) (width 0.381) (layer "F.Cu") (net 16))
 (segment (start 152.3111 79.6358) (end 152.3111 80.9031) (width 0.381) (layer "F.Cu") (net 16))
 (segment (start 152.3111 80.9031) (end 151.9642 81.25) (width 0.381) (layer "F.Cu") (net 16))
 (segment (start 143.3025 76.6075) (end 146.4025 76.6075) (width 0.381) (layer "F.Cu") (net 16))
 (segment (start 146.4025 76.6075) (end 146.4775 76.6825) (width 0.381) (layer "F.Cu") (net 16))
 (segment (start 150.5175 77.8422) (end 152.3111 79.6358) (width 0.381) (layer "F.Cu") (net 16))
 (segment (start 135.8622 82.4298) (end 135.8622 81.915) (width 0.381) (layer "F.Cu") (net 8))
 (segment (start 134.62 81.915) (end 135.8622 81.915) (width 0.381) (layer "F.Cu") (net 8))
 (segment (start 151.13 84.5) (end 148.6741 86.9559) (width 0.381) (layer "F.Cu") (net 8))
 (segment (start 137.6888 83.185) (end 136.6174 83.185) (width 0.381) (layer "F.Cu") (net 8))
 (segment (start 141.3502 86.9559) (end 139.3969 85.0026) (width 0.381) (layer "F.Cu") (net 8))
 (segment (start 151.315 84.685) (end 156.115 84.685) (width 0.381) (layer "F.Cu") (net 8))
 (segment (start 139.3969 85.0026) (end 139.3969 84.8931) (width 0.381) (layer "F.Cu") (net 8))
 (segment (start 151.13 84.5) (end 151.315 84.685) (width 0.381) (layer "F.Cu") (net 8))
 (segment (start 136.6174 83.185) (end 135.8622 82.4298) (width 0.381) (layer "F.Cu") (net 8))
 (segment (start 148.6741 86.9559) (end 141.3502 86.9559) (width 0.381) (layer "F.Cu") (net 8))
 (segment (start 139.3969 84.8931) (end 137.6888 83.185) (width 0.381) (layer "F.Cu") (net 8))
 (segment (start 141.7064 73.5934) (end 139.7349 75.5649) (width 0.381) (layer "F.Cu") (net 11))
 (segment (start 135.8622 76.3202) (end 135.8622 76.835) (width 0.381) (layer "F.Cu") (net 11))
 (segment (start 155.875 77.7) (end 154.2648 79.3102) (width 0.381) (layer "F.Cu") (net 11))
 (segment (start 152.6175 83.2) (end 151.13 83.2) (width 0.381) (layer "F.Cu") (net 11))
 (segment (start 154.2648 81.5527) (end 152.6175 83.2) (width 0.381) (layer "F.Cu") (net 11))
 (segment (start 154.2648 79.3102) (end 154.2648 81.5527) (width 0.381) (layer "F.Cu") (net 11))
 (segment (start 155.875 77.7) (end 151.7684 73.5934) (width 0.381) (layer "F.Cu") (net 11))
 (segment (start 151.7684 73.5934) (end 141.7064 73.5934) (width 0.381) (layer "F.Cu") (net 11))
 (segment (start 136.6175 75.5649) (end 135.8622 76.3202) (width 0.381) (layer "F.Cu") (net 11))
 (segment (start 139.7349 75.5649) (end 136.6175 75.5649) (width 0.381) (layer "F.Cu") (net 11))
 (segment (start 134.62 76.835) (end 135.8622 76.835) (width 0.381) (layer "F.Cu") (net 11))
 (segment (start 157.115 85.4249) (end 154.9492 87.5907) (width 0.381) (layer "F.Cu") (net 9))
 (segment (start 140.0104 87.5907) (end 138.1725 85.7528) (width 0.381) (layer "F.Cu") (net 9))
 (segment (start 135.9178 85.0212) (end 135.9178 83.6442) (width 0.381) (layer "F.Cu") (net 9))
 (segment (start 151.13 83.85) (end 154.8144 83.85) (width 0.381) (layer "F.Cu") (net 9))
 (segment (start 138.1725 85.7528) (end 136.6494 85.7528) (width 0.381) (layer "F.Cu") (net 9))
 (segment (start 154.9492 87.5907) (end 140.0104 87.5907) (width 0.381) (layer "F.Cu") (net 9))
 (segment (start 135.9178 83.6442) (end 135.7866 83.513) (width 0.381) (layer "F.Cu") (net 9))
 (segment (start 155.875 82.7894) (end 155.875 81.28) (width 0.381) (layer "F.Cu") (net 9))
 (segment (start 157.115 83.9752) (end 157.115 85.4249) (width 0.381) (layer "F.Cu") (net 9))
 (segment (start 155.875 82.7894) (end 155.9292 82.7894) (width 0.381) (layer "F.Cu") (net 9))
 (segment (start 154.8144 83.85) (end 155.875 82.7894) (width 0.381) (layer "F.Cu") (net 9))
 (segment (start 155.9292 82.7894) (end 157.115 83.9752) (width 0.381) (layer "F.Cu") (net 9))
 (segment (start 136.6494 85.7528) (end 135.9178 85.0212) (width 0.381) (layer "F.Cu") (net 9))
 (via (at 135.7866 83.513) (size 0.8) (drill 0.4) (layers "F.Cu" "B.Cu") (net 9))
 (segment (start 134.62 79.375) (end 134.62 80.6172) (width 0.381) (layer "B.Cu") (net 9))
 (segment (start 135.9178 83.3818) (end 135.7866 83.513) (width 0.381) (layer "B.Cu") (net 9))
 (segment (start 134.62 80.6172) (end 135.0858 80.6172) (width 0.381) (layer "B.Cu") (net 9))
 (segment (start 135.0858 80.6172) (end 135.9178 81.4492) (width 0.381) (layer "B.Cu") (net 9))
 (segment (start 135.9178 81.4492) (end 135.9178 83.3818) (width 0.381) (layer "B.Cu") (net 9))
 (segment (start 145.405 83.2) (end 144.5446 83.2) (width 0.381) (layer "F.Cu") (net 18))
 (segment (start 144.2237 83.5209) (end 144.2237 83.8761) (width 0.381) (layer "F.Cu") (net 18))
 (segment (start 144.5446 83.2) (end 144.2237 83.5209) (width 0.381) (layer "F.Cu") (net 18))
 (segment (start 144.2237 83.8761) (end 142.1248 85.975) (width 0.381) (layer "F.Cu") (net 18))
 (segment (start 143.4748 82.55) (end 145.405 82.55) (width 0.381) (layer "F.Cu") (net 17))
 (segment (start 142.1248 83.9) (end 143.4748 82.55) (width 0.381) (layer "F.Cu") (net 17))
 (segment (start 145.405 81.9) (end 142.4025 81.9) (width 0.381) (layer "F.Cu") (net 14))
 (segment (start 142.4025 81.9) (end 142.0325 81.53) (width 0.381) (layer "F.Cu") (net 14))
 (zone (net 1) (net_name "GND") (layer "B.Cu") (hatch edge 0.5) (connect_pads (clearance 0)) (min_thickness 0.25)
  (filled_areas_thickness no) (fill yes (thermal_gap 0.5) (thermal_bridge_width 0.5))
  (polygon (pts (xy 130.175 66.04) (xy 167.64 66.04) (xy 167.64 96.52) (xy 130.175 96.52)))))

